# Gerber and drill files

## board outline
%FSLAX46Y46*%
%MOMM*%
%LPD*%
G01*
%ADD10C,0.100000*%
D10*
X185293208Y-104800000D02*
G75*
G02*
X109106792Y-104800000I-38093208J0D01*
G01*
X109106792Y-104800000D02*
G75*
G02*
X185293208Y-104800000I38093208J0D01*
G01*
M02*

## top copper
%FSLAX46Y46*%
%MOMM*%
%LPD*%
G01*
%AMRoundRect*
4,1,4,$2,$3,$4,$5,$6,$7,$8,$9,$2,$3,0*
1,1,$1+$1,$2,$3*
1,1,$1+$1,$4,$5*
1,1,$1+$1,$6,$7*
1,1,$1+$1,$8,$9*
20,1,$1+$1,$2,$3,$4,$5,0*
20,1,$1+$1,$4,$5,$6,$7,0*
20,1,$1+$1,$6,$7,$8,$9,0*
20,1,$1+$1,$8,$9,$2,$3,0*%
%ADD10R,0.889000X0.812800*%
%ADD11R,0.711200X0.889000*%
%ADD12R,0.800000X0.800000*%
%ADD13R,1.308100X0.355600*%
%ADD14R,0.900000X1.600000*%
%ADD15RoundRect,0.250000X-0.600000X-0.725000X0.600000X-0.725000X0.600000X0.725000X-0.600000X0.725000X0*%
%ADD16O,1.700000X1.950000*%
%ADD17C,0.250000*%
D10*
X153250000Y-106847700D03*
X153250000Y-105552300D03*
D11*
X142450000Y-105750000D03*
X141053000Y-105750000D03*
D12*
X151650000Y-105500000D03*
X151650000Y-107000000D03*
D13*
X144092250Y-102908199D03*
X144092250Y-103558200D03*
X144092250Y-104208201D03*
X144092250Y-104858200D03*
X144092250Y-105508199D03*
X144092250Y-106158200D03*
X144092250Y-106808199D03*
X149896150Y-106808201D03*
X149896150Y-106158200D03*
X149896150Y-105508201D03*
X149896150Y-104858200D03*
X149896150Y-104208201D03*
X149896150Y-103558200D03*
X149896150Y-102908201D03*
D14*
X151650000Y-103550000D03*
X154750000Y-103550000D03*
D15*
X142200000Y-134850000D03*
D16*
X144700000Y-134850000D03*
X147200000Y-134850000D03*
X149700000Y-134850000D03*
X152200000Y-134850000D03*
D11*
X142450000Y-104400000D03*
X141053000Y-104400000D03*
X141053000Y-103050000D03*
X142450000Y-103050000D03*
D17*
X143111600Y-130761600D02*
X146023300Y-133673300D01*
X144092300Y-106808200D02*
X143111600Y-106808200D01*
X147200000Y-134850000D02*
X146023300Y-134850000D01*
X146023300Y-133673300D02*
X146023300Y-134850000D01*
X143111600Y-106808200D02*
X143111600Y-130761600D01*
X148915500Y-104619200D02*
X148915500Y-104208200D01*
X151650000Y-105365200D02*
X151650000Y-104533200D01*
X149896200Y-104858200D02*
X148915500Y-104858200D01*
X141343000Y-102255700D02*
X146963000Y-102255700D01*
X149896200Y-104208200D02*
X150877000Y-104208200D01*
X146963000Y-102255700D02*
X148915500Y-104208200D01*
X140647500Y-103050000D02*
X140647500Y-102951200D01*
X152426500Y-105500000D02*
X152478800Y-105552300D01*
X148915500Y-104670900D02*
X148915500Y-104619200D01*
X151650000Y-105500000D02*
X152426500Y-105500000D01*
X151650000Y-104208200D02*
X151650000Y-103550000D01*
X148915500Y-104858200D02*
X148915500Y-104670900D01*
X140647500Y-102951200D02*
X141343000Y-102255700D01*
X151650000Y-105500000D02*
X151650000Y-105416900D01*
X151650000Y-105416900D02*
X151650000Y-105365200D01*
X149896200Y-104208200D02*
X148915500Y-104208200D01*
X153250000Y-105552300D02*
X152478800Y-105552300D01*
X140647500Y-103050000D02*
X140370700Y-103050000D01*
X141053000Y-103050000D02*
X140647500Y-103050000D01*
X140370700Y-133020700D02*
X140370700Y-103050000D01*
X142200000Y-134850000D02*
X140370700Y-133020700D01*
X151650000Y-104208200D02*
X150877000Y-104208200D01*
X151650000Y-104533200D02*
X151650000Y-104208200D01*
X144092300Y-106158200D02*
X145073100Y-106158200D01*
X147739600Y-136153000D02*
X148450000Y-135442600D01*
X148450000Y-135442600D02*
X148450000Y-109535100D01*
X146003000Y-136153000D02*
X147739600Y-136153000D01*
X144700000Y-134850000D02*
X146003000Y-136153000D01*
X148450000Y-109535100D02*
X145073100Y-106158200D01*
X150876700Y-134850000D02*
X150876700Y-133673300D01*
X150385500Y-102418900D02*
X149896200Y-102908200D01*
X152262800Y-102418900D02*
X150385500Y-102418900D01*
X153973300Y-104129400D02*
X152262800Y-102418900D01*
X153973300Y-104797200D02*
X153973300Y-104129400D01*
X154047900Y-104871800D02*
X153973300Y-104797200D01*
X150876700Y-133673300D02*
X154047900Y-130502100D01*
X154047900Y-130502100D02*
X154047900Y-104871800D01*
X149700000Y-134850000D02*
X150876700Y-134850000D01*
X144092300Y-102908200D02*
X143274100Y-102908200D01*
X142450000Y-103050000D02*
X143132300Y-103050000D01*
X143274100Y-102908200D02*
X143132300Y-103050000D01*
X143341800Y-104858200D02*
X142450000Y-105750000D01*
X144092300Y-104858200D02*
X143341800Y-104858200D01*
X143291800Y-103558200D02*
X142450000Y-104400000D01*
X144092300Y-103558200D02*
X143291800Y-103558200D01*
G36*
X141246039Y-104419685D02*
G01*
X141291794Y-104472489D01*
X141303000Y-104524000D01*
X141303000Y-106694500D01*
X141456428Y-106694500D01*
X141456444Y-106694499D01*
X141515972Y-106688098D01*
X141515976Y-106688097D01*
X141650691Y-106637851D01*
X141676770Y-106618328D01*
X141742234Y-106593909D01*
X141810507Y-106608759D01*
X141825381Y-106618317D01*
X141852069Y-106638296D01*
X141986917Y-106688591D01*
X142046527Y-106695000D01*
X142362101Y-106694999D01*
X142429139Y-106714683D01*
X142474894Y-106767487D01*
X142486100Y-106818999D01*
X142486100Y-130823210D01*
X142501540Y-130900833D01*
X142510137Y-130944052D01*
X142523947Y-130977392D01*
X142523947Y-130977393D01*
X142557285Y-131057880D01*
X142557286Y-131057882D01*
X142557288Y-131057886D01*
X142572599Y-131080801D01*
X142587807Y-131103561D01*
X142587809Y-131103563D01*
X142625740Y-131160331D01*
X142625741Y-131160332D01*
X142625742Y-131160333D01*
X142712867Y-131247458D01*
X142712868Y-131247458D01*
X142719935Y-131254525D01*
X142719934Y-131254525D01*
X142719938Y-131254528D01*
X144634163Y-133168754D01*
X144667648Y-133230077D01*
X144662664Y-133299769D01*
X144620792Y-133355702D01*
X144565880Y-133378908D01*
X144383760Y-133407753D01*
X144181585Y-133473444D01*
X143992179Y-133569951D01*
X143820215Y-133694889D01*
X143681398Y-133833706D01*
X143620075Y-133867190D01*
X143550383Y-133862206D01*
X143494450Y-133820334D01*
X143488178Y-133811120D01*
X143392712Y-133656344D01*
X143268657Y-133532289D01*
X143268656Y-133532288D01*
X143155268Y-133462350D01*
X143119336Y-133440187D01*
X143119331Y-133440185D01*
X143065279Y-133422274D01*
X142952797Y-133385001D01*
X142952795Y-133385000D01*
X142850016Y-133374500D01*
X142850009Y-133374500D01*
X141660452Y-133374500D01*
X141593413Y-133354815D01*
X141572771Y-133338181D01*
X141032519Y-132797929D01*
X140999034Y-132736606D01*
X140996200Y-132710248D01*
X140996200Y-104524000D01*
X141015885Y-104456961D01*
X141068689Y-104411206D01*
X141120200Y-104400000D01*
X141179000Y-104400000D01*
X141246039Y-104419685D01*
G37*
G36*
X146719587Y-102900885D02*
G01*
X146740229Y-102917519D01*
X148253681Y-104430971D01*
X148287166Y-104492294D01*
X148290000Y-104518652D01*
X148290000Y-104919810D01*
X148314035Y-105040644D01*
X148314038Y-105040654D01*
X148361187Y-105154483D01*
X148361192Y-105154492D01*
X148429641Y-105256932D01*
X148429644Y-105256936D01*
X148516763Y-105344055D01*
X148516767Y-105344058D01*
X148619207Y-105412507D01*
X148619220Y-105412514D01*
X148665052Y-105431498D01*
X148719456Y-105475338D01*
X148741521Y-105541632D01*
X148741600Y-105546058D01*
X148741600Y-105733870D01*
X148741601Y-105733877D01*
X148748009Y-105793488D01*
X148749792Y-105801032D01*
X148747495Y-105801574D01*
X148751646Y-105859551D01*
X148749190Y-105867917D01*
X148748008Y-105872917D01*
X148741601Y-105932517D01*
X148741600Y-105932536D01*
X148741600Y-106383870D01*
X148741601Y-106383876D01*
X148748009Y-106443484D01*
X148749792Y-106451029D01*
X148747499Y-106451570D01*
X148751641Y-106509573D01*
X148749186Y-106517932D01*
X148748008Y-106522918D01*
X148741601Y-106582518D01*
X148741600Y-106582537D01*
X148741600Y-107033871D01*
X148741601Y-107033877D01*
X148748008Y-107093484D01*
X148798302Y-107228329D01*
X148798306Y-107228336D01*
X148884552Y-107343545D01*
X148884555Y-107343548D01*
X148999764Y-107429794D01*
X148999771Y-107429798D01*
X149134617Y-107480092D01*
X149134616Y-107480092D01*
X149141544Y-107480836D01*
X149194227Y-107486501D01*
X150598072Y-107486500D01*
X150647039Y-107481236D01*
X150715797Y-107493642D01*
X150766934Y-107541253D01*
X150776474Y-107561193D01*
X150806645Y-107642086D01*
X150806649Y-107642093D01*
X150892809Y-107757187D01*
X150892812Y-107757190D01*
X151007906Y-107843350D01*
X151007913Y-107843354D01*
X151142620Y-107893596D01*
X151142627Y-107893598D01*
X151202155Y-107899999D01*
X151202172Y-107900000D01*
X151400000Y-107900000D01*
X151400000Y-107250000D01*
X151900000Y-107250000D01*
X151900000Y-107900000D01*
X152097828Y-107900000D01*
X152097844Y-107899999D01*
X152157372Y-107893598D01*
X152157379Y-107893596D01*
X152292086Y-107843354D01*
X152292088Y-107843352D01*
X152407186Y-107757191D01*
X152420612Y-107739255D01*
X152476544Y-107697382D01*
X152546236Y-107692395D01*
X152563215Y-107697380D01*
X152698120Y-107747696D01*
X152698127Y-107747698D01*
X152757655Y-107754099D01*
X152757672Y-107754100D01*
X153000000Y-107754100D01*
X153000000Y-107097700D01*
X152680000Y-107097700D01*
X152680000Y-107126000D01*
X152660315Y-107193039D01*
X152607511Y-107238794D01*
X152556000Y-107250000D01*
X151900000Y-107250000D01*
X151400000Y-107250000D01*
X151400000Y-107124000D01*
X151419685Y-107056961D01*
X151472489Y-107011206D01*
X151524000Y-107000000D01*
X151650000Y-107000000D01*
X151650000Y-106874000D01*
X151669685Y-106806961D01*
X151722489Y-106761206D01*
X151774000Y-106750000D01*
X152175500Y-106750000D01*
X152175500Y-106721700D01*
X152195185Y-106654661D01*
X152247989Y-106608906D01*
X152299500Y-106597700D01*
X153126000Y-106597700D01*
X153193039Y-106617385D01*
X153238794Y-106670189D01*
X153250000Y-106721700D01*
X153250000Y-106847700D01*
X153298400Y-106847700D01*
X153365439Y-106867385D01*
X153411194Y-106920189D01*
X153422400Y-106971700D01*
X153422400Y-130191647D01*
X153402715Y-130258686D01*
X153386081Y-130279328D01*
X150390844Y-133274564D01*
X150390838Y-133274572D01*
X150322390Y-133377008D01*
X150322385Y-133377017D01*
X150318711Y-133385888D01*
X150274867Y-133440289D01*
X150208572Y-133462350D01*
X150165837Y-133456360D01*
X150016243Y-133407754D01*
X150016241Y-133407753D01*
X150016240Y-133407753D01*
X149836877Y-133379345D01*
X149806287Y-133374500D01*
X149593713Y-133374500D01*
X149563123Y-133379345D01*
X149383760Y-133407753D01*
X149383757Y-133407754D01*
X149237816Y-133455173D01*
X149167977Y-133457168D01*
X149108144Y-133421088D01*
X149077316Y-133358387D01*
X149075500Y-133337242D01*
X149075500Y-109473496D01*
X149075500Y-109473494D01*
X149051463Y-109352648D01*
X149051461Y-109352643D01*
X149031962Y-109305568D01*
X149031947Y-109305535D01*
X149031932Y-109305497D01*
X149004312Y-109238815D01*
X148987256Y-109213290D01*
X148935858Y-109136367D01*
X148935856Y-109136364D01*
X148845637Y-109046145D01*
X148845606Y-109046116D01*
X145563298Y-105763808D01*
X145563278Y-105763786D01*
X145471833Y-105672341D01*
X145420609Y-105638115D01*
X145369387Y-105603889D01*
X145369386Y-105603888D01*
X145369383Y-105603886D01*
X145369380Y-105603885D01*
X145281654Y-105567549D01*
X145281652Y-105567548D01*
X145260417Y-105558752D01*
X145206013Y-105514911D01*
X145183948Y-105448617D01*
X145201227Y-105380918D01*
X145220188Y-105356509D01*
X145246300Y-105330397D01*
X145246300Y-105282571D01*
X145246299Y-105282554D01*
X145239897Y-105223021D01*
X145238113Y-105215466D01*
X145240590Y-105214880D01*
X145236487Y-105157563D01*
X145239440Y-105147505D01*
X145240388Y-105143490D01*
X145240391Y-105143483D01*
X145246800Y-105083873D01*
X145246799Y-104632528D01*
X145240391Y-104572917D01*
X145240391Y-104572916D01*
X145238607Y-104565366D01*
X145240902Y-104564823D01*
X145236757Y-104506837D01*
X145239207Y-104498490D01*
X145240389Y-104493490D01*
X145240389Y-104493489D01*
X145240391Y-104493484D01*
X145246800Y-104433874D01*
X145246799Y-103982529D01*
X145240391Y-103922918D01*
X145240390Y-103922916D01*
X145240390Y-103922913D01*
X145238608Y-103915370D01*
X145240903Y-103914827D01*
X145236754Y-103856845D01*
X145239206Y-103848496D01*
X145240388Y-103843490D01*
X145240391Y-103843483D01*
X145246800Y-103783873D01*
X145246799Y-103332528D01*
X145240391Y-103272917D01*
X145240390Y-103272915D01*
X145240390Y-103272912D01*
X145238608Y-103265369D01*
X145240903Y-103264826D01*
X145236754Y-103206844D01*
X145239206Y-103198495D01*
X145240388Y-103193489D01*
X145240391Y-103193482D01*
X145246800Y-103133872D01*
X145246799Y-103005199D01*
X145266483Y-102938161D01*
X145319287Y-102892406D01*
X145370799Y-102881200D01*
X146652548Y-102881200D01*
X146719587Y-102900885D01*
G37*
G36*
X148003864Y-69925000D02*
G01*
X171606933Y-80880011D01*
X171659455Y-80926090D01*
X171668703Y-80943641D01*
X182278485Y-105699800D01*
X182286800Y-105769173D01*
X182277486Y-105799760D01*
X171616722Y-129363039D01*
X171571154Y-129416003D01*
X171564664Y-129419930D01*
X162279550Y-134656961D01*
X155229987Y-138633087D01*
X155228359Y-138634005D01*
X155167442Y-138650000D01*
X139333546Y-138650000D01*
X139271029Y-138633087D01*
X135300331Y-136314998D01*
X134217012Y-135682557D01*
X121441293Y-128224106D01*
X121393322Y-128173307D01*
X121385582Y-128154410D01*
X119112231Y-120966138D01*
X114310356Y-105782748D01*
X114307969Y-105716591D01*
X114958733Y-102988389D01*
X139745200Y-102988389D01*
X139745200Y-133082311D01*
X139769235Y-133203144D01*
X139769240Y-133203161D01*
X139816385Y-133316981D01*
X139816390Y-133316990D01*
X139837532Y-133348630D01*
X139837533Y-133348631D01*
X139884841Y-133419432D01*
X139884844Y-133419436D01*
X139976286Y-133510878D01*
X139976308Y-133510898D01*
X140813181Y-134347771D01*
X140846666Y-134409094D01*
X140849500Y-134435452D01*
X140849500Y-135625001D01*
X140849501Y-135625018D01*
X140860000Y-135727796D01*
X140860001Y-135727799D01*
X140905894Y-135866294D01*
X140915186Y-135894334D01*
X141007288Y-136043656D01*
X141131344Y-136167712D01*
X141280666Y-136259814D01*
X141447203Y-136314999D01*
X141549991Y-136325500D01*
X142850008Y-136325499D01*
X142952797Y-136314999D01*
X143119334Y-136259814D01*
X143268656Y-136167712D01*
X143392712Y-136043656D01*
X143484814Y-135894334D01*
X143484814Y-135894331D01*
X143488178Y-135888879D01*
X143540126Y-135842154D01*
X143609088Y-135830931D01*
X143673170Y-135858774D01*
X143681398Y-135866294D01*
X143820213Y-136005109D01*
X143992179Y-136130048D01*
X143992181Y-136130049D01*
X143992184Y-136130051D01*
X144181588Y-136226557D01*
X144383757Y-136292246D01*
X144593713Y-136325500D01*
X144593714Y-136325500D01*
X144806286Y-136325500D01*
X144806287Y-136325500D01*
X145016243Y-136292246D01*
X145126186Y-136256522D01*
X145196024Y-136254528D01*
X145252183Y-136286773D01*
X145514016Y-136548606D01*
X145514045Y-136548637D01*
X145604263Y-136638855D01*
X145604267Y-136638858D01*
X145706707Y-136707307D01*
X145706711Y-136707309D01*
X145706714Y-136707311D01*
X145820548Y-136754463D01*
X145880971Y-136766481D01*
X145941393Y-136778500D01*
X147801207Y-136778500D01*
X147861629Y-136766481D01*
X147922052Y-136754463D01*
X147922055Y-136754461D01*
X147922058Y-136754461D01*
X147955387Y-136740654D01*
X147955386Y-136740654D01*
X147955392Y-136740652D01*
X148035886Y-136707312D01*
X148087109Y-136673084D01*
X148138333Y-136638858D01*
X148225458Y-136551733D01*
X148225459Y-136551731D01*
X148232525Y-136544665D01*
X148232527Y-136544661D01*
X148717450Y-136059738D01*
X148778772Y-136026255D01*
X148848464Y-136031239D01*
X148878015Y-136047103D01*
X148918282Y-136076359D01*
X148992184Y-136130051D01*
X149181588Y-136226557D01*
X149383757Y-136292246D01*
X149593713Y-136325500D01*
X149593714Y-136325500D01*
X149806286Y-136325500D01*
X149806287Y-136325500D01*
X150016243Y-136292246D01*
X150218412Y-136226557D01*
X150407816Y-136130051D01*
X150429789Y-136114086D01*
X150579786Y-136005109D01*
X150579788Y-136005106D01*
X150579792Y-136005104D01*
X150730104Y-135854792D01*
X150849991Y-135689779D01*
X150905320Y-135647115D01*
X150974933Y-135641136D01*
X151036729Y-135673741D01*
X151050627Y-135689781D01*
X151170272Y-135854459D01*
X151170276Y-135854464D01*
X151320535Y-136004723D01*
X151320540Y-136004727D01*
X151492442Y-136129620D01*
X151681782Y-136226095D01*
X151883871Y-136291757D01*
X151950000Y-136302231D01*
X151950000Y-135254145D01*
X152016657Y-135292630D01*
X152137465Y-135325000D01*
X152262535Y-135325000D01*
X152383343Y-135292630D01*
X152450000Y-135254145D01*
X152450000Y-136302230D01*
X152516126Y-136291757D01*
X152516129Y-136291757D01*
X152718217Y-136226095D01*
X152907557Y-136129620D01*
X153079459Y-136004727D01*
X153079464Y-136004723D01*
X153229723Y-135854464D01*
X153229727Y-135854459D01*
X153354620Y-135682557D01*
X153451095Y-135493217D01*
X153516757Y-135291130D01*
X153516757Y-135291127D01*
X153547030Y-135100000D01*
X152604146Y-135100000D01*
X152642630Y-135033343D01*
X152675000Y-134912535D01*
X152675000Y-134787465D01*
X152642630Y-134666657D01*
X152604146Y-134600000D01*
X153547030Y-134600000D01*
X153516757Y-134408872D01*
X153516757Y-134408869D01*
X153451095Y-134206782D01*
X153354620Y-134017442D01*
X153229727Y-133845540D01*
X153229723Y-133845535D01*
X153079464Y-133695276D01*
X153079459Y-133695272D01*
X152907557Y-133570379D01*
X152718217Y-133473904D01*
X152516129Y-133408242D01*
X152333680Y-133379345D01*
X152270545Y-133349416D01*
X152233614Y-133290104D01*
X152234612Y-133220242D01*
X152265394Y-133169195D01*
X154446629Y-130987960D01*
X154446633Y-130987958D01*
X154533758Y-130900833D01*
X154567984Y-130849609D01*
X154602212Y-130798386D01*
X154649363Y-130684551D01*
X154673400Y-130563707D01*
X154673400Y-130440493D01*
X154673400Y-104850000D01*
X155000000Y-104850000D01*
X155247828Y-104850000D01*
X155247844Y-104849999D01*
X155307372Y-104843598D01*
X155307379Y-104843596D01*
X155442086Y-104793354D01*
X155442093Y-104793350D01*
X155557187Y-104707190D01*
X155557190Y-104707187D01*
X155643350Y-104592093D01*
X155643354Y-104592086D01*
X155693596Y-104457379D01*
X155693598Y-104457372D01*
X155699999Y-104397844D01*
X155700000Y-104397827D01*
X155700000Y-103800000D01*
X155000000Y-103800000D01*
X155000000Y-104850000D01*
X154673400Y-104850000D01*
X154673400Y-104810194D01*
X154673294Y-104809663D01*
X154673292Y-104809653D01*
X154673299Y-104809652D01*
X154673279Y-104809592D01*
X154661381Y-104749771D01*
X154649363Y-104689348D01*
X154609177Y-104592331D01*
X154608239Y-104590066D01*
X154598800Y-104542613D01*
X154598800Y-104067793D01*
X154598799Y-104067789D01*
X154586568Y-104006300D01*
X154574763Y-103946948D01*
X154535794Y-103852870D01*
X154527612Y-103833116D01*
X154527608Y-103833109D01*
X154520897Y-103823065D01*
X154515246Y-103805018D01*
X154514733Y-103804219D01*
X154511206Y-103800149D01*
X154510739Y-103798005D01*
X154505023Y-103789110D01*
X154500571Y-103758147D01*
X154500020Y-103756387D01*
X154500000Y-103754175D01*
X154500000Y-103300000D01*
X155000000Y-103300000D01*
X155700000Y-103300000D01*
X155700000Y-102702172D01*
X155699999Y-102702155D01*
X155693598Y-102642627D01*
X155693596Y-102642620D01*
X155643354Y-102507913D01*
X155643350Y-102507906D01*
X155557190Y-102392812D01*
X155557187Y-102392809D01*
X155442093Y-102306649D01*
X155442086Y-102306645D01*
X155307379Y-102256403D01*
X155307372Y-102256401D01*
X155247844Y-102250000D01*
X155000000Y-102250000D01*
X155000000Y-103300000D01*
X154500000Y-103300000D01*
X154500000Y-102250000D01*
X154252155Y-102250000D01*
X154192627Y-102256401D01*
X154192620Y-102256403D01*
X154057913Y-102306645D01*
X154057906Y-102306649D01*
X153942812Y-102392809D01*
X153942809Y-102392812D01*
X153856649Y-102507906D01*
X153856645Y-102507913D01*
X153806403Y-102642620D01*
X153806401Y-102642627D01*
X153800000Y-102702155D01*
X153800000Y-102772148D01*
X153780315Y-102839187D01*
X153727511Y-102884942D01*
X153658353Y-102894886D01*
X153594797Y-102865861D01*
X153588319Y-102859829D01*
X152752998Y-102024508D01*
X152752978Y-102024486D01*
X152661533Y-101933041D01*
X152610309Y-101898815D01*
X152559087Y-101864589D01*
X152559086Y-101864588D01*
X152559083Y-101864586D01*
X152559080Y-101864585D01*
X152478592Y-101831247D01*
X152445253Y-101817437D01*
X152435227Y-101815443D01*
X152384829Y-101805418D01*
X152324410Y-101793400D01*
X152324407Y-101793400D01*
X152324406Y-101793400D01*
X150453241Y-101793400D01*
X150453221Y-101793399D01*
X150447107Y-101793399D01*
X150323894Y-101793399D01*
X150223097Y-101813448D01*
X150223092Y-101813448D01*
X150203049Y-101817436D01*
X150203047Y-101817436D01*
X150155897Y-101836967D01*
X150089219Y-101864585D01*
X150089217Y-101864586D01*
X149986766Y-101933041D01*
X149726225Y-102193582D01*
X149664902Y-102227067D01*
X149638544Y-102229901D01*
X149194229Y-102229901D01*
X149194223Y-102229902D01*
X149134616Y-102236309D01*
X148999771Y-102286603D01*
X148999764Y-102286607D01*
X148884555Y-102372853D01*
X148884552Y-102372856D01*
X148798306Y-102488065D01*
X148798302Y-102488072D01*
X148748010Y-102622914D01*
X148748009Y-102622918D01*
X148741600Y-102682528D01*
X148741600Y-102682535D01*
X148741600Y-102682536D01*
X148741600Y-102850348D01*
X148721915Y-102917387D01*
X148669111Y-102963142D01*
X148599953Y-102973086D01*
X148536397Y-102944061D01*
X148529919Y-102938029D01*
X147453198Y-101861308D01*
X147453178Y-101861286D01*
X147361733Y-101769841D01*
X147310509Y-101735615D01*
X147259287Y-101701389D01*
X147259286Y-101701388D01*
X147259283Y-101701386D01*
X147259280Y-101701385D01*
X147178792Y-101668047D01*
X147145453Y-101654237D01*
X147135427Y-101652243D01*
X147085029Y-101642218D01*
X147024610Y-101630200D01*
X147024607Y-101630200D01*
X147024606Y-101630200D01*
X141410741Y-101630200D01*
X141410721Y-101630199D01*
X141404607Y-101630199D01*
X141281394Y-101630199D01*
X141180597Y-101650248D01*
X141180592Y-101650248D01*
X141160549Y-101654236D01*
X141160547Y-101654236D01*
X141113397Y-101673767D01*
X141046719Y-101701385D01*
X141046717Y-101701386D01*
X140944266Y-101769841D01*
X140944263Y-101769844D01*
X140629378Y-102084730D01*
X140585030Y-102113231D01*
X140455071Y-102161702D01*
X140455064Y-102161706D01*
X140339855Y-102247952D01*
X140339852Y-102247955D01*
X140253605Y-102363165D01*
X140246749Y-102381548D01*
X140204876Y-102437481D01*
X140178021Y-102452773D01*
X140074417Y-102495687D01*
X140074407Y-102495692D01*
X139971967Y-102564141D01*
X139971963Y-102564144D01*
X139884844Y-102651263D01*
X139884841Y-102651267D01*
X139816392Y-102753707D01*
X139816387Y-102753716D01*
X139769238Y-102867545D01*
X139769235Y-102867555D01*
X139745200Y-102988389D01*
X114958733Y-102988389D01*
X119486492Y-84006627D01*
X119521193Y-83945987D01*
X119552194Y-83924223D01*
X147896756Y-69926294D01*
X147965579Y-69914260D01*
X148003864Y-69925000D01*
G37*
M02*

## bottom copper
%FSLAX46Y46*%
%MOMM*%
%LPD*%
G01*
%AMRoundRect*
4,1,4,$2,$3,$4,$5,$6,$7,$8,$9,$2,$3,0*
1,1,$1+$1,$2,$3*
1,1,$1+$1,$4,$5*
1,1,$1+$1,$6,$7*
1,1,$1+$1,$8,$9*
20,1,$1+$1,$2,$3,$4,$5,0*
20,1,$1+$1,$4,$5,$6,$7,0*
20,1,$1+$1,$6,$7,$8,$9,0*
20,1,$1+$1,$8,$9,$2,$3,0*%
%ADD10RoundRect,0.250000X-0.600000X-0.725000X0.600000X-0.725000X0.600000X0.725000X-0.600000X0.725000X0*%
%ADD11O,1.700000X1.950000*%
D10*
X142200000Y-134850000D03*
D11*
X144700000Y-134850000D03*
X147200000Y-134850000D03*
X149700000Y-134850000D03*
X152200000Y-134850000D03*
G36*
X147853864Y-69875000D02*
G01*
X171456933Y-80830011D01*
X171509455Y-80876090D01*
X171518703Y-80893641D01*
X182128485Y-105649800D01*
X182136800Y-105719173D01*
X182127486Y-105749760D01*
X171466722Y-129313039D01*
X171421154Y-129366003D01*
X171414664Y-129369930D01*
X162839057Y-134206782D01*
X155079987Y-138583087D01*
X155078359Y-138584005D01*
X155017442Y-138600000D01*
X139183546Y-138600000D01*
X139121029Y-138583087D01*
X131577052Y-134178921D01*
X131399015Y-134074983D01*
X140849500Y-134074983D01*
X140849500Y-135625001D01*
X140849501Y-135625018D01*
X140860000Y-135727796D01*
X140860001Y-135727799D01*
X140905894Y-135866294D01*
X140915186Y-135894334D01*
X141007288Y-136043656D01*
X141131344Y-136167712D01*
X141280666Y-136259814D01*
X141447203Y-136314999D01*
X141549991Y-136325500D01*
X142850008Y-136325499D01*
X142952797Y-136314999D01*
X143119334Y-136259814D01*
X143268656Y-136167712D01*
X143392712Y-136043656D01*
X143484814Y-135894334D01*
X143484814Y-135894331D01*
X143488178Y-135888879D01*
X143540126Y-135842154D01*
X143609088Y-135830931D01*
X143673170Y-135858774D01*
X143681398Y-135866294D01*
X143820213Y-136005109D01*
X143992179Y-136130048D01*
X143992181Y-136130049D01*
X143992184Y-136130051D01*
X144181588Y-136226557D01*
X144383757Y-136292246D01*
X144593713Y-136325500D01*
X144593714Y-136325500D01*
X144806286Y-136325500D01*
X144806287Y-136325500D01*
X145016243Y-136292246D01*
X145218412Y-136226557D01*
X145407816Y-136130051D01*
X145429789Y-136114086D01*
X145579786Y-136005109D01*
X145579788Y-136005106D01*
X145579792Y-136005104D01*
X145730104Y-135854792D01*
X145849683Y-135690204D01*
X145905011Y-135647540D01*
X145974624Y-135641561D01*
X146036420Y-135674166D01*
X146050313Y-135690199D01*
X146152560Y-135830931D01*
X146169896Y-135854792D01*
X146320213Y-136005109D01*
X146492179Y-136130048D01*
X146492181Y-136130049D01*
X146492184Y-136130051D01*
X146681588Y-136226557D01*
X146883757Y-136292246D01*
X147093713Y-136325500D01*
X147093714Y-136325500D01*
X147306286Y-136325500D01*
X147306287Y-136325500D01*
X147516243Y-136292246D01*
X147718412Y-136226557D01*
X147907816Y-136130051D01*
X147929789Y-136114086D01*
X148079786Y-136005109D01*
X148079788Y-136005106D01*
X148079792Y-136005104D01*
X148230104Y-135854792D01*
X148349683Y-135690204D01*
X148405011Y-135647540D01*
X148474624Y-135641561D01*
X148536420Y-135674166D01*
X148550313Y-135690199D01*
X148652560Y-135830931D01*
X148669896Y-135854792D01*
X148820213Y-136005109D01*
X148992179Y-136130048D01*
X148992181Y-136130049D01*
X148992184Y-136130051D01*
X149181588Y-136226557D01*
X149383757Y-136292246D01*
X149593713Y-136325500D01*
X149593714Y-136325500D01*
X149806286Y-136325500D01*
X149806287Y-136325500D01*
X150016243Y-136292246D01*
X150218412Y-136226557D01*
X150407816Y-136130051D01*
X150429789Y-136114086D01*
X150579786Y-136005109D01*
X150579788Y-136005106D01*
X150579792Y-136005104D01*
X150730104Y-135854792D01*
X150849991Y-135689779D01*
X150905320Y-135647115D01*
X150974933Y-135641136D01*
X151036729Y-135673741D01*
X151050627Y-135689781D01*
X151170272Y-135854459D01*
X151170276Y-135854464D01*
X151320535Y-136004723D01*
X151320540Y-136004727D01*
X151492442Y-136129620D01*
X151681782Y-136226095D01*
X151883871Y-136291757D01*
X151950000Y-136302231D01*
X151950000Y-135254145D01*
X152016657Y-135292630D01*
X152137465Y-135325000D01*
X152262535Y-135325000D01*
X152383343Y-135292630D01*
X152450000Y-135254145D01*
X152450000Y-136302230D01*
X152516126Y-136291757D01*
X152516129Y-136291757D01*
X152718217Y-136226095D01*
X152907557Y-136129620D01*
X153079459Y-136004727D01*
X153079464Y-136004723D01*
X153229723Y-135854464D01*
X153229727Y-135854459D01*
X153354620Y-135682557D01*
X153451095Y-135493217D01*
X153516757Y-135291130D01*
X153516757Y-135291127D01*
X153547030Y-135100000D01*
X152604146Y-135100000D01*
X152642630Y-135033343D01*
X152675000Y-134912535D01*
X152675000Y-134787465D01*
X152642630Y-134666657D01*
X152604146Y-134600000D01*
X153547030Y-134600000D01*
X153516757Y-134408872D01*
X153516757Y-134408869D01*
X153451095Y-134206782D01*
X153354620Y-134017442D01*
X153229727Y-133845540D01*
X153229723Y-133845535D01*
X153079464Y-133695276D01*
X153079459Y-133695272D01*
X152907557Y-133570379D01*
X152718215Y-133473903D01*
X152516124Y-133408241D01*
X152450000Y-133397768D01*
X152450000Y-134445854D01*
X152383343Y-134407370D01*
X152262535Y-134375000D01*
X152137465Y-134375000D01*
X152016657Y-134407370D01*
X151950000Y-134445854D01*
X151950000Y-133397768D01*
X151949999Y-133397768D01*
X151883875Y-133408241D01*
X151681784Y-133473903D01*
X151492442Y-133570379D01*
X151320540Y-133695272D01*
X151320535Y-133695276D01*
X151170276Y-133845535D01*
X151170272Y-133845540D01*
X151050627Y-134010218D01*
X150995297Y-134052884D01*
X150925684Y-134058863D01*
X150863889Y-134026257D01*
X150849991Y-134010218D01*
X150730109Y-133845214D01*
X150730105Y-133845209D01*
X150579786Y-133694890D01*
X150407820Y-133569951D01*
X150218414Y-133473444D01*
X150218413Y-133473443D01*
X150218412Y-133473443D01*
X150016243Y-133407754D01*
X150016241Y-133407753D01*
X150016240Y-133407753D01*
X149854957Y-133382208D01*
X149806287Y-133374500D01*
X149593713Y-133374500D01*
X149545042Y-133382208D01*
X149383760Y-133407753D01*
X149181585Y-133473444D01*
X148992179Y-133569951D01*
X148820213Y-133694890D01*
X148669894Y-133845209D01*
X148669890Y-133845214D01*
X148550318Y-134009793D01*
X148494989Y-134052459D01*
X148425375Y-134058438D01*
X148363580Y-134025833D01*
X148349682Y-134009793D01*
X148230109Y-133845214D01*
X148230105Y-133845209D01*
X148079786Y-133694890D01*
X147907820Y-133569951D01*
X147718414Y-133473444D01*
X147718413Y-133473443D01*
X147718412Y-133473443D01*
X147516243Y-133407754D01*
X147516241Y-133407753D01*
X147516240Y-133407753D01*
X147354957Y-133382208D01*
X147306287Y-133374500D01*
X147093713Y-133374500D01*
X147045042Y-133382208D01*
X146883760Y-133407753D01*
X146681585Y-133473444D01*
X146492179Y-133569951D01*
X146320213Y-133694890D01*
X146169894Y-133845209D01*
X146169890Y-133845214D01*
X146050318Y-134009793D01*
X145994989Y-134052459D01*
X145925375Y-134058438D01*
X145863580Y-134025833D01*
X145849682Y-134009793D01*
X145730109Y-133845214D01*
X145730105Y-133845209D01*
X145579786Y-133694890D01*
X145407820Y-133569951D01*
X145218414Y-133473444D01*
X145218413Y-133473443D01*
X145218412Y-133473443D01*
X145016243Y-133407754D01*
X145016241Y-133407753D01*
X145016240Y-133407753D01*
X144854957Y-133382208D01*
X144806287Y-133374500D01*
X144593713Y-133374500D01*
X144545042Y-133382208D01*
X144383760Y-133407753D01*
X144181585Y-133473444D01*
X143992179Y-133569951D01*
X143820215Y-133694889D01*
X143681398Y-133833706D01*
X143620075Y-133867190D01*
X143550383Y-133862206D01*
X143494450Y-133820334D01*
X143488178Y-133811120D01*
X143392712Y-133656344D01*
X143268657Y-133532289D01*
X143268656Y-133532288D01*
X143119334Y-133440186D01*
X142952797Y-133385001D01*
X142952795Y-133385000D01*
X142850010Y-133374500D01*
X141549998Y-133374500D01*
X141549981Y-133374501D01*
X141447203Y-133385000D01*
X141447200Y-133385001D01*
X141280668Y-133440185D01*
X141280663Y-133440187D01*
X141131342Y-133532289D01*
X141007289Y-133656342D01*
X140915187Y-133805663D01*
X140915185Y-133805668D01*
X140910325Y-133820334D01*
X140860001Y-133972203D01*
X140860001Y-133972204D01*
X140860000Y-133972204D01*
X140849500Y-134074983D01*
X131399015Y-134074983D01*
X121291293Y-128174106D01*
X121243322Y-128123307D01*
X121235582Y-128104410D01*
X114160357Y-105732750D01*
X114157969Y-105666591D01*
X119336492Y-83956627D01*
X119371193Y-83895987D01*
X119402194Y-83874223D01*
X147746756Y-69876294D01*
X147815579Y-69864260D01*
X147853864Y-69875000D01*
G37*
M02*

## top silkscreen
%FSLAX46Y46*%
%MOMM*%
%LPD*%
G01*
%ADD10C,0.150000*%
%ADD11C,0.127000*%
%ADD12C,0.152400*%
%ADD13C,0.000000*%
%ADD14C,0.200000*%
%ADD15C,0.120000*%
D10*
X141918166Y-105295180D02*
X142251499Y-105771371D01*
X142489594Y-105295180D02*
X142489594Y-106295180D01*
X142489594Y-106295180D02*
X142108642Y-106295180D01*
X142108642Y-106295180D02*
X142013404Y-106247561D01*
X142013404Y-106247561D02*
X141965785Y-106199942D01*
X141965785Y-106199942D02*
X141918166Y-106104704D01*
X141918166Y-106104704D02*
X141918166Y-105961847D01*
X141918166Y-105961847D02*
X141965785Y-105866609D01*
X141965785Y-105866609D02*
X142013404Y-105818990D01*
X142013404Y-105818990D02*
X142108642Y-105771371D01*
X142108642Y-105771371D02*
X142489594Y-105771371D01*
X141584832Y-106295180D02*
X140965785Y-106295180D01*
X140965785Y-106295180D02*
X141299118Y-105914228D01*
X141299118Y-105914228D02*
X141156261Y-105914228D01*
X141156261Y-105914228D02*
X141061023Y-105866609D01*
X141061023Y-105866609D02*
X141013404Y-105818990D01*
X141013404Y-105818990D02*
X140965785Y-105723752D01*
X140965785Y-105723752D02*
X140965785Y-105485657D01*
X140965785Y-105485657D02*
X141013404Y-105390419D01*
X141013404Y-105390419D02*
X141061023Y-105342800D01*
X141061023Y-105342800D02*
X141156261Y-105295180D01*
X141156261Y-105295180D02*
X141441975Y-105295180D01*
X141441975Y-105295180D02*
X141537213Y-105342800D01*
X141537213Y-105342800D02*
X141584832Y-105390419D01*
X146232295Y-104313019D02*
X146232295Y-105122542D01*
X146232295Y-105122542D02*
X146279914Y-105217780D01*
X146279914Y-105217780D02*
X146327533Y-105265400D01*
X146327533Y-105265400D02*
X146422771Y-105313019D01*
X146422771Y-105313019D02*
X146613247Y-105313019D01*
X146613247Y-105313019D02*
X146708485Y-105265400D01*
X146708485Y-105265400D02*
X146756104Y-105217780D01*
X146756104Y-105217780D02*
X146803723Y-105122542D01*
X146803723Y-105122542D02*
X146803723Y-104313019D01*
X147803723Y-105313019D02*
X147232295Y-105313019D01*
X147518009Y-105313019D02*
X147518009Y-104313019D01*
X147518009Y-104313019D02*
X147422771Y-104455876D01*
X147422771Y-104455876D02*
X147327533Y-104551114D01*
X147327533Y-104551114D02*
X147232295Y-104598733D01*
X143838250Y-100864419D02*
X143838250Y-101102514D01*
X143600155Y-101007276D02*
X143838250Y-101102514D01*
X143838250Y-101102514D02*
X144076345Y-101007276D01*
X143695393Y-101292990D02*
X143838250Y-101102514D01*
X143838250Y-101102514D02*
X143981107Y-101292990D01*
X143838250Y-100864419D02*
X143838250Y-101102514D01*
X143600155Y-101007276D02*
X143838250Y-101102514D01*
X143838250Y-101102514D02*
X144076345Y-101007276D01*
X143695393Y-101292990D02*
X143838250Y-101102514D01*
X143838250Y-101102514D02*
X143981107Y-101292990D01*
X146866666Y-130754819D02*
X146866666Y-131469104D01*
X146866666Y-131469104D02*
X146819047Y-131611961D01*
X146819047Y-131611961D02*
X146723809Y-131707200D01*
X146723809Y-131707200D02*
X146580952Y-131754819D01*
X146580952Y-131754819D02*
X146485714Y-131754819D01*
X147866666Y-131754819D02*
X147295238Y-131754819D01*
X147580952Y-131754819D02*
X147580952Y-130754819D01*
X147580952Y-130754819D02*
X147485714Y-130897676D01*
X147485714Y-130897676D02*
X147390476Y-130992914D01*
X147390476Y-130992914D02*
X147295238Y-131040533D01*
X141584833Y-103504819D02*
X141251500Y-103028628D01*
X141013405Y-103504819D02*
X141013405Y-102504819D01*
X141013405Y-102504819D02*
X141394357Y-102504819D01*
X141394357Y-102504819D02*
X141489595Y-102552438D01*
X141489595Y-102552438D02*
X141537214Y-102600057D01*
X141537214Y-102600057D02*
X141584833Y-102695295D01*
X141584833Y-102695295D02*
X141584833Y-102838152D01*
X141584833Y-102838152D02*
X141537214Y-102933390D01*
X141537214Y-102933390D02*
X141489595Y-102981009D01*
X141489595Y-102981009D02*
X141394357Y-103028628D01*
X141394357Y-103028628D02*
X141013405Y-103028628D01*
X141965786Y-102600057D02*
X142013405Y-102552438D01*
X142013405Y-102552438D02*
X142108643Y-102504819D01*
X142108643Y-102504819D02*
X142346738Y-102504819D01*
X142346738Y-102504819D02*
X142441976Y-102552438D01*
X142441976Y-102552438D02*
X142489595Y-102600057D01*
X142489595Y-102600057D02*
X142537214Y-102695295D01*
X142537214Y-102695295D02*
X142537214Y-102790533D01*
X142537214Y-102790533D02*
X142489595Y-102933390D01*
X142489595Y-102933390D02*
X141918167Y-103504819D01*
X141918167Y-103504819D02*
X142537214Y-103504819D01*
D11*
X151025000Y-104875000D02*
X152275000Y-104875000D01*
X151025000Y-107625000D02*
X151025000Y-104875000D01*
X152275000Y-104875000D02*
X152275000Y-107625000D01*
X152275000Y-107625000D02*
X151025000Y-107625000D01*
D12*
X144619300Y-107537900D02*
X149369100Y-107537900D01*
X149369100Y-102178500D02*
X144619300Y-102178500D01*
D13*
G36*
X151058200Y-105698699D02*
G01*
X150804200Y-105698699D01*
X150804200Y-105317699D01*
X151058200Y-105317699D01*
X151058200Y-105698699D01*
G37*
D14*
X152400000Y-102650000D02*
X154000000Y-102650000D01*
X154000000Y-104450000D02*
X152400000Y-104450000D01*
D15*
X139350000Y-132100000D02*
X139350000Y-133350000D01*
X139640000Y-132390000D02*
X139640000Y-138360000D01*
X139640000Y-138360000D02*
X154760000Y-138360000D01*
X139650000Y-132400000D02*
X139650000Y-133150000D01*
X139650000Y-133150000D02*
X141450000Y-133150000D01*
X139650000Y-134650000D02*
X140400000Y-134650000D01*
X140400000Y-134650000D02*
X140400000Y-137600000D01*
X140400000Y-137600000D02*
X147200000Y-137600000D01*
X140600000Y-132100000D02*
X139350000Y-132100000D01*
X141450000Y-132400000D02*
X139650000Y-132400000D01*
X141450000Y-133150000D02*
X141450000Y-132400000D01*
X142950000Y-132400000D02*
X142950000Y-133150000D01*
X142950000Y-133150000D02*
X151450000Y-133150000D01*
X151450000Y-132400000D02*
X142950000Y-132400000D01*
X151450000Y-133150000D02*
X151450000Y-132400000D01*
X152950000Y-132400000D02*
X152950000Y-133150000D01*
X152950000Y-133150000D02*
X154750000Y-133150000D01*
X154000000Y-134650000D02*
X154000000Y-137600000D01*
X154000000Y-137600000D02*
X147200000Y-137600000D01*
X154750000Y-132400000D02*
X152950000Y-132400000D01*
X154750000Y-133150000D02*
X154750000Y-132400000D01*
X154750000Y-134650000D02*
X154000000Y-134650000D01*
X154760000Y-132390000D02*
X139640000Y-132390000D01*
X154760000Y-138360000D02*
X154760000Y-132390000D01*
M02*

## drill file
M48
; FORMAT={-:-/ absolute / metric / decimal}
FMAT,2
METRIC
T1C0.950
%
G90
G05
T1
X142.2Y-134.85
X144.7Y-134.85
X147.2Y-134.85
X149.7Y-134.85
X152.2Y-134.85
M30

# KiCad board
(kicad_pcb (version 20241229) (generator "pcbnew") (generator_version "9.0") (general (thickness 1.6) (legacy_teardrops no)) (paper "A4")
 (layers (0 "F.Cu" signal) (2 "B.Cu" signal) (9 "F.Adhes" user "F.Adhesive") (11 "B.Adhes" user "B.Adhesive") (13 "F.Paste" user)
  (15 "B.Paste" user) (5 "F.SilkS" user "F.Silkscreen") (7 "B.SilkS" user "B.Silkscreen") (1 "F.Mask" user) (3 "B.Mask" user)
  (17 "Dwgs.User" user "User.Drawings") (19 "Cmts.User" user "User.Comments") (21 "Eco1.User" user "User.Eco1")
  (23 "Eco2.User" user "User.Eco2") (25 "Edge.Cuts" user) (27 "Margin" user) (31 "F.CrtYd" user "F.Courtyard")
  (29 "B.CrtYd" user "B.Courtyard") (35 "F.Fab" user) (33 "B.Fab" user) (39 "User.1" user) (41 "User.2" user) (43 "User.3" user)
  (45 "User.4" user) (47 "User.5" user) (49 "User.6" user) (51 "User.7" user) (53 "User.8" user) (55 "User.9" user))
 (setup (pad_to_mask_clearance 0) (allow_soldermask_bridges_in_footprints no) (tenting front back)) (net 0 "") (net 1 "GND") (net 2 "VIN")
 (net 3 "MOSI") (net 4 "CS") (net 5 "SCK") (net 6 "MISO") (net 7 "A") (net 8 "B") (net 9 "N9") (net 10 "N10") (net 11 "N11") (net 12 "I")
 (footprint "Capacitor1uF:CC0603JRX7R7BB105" (layer "F.Cu") (at 153.25 106.2 90)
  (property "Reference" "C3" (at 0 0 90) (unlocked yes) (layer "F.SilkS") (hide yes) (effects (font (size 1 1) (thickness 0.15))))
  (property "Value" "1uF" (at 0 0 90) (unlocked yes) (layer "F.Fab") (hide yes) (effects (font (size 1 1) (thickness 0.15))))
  (pad "1" smd rect (at -0.6477 0 90) (size 0.8128 0.889) (layers "F.Cu" "F.Mask" "F.Paste") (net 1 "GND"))
  (pad "2" smd rect (at 0.6477 0 90) (size 0.8128 0.889) (layers "F.Cu" "F.Mask" "F.Paste") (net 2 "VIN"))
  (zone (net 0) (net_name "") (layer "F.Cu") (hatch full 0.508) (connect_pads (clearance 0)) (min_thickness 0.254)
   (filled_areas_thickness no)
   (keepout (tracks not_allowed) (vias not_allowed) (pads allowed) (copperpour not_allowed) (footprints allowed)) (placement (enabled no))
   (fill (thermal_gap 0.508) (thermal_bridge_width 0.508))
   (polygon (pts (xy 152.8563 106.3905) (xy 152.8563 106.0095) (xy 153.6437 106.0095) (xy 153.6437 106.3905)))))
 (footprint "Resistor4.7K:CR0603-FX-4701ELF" (layer "F.Cu") (at 141.7515 105.75 180)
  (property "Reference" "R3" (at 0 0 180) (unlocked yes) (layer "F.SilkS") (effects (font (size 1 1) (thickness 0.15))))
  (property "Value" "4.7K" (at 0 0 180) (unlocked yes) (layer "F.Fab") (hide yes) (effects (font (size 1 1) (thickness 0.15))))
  (pad "1" smd rect (at -0.6985 0 180) (size 0.7112 0.889) (layers "F.Cu" "F.Mask" "F.Paste") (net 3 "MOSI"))
  (pad "2" smd rect (at 0.6985 0 180) (size 0.7112 0.889) (layers "F.Cu" "F.Mask" "F.Paste") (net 1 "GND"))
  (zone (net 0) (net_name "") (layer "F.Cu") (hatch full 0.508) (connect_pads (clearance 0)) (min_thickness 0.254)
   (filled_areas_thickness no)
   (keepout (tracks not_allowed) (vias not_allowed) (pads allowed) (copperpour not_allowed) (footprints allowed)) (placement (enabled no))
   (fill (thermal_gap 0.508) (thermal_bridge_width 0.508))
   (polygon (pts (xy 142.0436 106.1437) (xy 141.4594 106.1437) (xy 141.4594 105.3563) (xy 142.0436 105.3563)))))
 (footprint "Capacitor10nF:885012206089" (layer "F.Cu") (at 151.65 106.25 -90)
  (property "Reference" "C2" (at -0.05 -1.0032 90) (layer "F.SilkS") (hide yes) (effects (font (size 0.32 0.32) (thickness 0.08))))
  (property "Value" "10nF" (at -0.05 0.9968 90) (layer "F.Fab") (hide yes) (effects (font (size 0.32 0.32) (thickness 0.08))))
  (fp_line (start -1.375 0.625) (end -1.375 -0.625) (stroke (width 0.127) (type solid)) (layer "F.SilkS"))
  (fp_line (start 1.375 0.625) (end -1.375 0.625) (stroke (width 0.127) (type solid)) (layer "F.SilkS"))
  (fp_line (start -1.375 -0.625) (end 1.375 -0.625) (stroke (width 0.127) (type solid)) (layer "F.SilkS"))
  (fp_line (start 1.375 -0.625) (end 1.375 0.625) (stroke (width 0.127) (type solid)) (layer "F.SilkS"))
  (pad "1" smd rect (at -0.75 0 270) (size 0.8 0.8) (layers "F.Cu" "F.Mask" "F.Paste") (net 2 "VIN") (solder_mask_margin 0.102))
  (pad "2" smd rect (at 0.75 0 270) (size 0.8 0.8) (layers "F.Cu" "F.Mask" "F.Paste") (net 1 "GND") (solder_mask_margin 0.102)))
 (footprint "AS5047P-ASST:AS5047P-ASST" (layer "F.Cu") (at 146.9942 104.8582)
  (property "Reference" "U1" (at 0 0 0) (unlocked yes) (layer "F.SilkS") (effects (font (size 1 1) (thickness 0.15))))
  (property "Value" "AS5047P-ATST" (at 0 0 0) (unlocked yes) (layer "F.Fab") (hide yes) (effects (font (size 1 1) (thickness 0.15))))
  (fp_line (start -2.3749 2.6797) (end 2.3749 2.6797) (stroke (width 0.1524) (type solid)) (layer "F.SilkS"))
  (fp_line (start 2.3749 -2.6797) (end -2.3749 -2.6797) (stroke (width 0.1524) (type solid)) (layer "F.SilkS"))
  (fp_poly
   (pts (xy 4.064 0.459499) (xy 4.064 0.840499) (xy 3.81 0.840499) (xy 3.81 0.459499)) (stroke (width 0) (type solid)) (fill yes)
   (layer "F.SilkS"))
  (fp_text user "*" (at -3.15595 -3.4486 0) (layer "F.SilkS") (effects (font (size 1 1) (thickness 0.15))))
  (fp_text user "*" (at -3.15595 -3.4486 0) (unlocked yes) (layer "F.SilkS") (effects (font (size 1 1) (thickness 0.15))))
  (pad "1" smd rect (at -2.90195 -1.950001) (size 1.3081 0.3556) (layers "F.Cu" "F.Mask" "F.Paste") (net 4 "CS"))
  (pad "2" smd rect (at -2.90195 -1.3) (size 1.3081 0.3556) (layers "F.Cu" "F.Mask" "F.Paste") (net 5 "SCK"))
  (pad "3" smd rect (at -2.90195 -0.649999) (size 1.3081 0.3556) (layers "F.Cu" "F.Mask" "F.Paste") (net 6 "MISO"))
  (pad "4" smd rect (at -2.90195 0) (size 1.3081 0.3556) (layers "F.Cu" "F.Mask" "F.Paste") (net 3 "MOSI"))
  (pad "5" smd rect (at -2.90195 0.649999) (size 1.3081 0.3556) (layers "F.Cu" "F.Mask" "F.Paste") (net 1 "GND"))
  (pad "6" smd rect (at -2.90195 1.3) (size 1.3081 0.3556) (layers "F.Cu" "F.Mask" "F.Paste") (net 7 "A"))
  (pad "7" smd rect (at -2.90195 1.949999) (size 1.3081 0.3556) (layers "F.Cu" "F.Mask" "F.Paste") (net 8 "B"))
  (pad "8" smd rect (at 2.90195 1.950001) (size 1.3081 0.3556) (layers "F.Cu" "F.Mask" "F.Paste") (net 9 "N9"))
  (pad "9" smd rect (at 2.90195 1.3) (size 1.3081 0.3556) (layers "F.Cu" "F.Mask" "F.Paste") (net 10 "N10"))
  (pad "10" smd rect (at 2.90195 0.650001) (size 1.3081 0.3556) (layers "F.Cu" "F.Mask" "F.Paste") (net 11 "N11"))
  (pad "11" smd rect (at 2.90195 0) (size 1.3081 0.3556) (layers "F.Cu" "F.Mask" "F.Paste") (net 2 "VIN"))
  (pad "12" smd rect (at 2.90195 -0.649999) (size 1.3081 0.3556) (layers "F.Cu" "F.Mask" "F.Paste") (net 2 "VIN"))
  (pad "13" smd rect (at 2.90195 -1.3) (size 1.3081 0.3556) (layers "F.Cu" "F.Mask" "F.Paste") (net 1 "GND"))
  (pad "14" smd rect (at 2.90195 -1.949999) (size 1.3081 0.3556) (layers "F.Cu" "F.Mask" "F.Paste") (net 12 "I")))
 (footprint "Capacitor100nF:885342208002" (layer "F.Cu") (at 153.2 103.55)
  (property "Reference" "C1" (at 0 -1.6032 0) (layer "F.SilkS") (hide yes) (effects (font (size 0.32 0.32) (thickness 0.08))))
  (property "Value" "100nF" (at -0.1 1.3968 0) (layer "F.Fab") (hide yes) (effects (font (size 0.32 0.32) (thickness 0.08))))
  (fp_line (start -0.8 -0.9) (end 0.8 -0.9) (stroke (width 0.2) (type solid)) (layer "F.SilkS"))
  (fp_line (start 0.8 0.9) (end -0.8 0.9) (stroke (width 0.2) (type solid)) (layer "F.SilkS"))
  (pad "1" smd rect (at -1.55 0) (size 0.9 1.6) (layers "F.Cu" "F.Mask" "F.Paste") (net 2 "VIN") (solder_mask_margin 0.102))
  (pad "2" smd rect (at 1.55 0) (size 0.9 1.6) (layers "F.Cu" "F.Mask" "F.Paste") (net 1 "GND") (solder_mask_margin 0.102)))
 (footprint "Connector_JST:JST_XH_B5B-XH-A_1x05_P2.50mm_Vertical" (layer "F.Cu") (at 142.2 134.85)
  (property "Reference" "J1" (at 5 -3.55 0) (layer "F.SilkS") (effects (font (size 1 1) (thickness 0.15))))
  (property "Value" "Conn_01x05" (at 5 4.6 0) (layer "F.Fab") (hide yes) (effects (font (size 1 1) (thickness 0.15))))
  (fp_line (start -2.85 -2.75) (end -2.85 -1.5) (stroke (width 0.12) (type solid)) (layer "F.SilkS"))
  (fp_line (start -2.56 -2.46) (end -2.56 3.51) (stroke (width 0.12) (type solid)) (layer "F.SilkS"))
  (fp_line (start -2.56 3.51) (end 12.56 3.51) (stroke (width 0.12) (type solid)) (layer "F.SilkS"))
  (fp_line (start -2.55 -2.45) (end -2.55 -1.7) (stroke (width 0.12) (type solid)) (layer "F.SilkS"))
  (fp_line (start -2.55 -1.7) (end -0.75 -1.7) (stroke (width 0.12) (type solid)) (layer "F.SilkS"))
  (fp_line (start -2.55 -0.2) (end -1.8 -0.2) (stroke (width 0.12) (type solid)) (layer "F.SilkS"))
  (fp_line (start -1.8 -0.2) (end -1.8 2.75) (stroke (width 0.12) (type solid)) (layer "F.SilkS"))
  (fp_line (start -1.8 2.75) (end 5 2.75) (stroke (width 0.12) (type solid)) (layer "F.SilkS"))
  (fp_line (start -1.6 -2.75) (end -2.85 -2.75) (stroke (width 0.12) (type solid)) (layer "F.SilkS"))
  (fp_line (start -0.75 -2.45) (end -2.55 -2.45) (stroke (width 0.12) (type solid)) (layer "F.SilkS"))
  (fp_line (start -0.75 -1.7) (end -0.75 -2.45) (stroke (width 0.12) (type solid)) (layer "F.SilkS"))
  (fp_line (start 0.75 -2.45) (end 0.75 -1.7) (stroke (width 0.12) (type solid)) (layer "F.SilkS"))
  (fp_line (start 0.75 -1.7) (end 9.25 -1.7) (stroke (width 0.12) (type solid)) (layer "F.SilkS"))
  (fp_line (start 9.25 -2.45) (end 0.75 -2.45) (stroke (width 0.12) (type solid)) (layer "F.SilkS"))
  (fp_line (start 9.25 -1.7) (end 9.25 -2.45) (stroke (width 0.12) (type solid)) (layer "F.SilkS"))
  (fp_line (start 10.75 -2.45) (end 10.75 -1.7) (stroke (width 0.12) (type solid)) (layer "F.SilkS"))
  (fp_line (start 10.75 -1.7) (end 12.55 -1.7) (stroke (width 0.12) (type solid)) (layer "F.SilkS"))
  (fp_line (start 11.8 -0.2) (end 11.8 2.75) (stroke (width 0.12) (type solid)) (layer "F.SilkS"))
  (fp_line (start 11.8 2.75) (end 5 2.75) (stroke (width 0.12) (type solid)) (layer "F.SilkS"))
  (fp_line (start 12.55 -2.45) (end 10.75 -2.45) (stroke (width 0.12) (type solid)) (layer "F.SilkS"))
  (fp_line (start 12.55 -1.7) (end 12.55 -2.45) (stroke (width 0.12) (type solid)) (layer "F.SilkS"))
  (fp_line (start 12.55 -0.2) (end 11.8 -0.2) (stroke (width 0.12) (type solid)) (layer "F.SilkS"))
  (fp_line (start 12.56 -2.46) (end -2.56 -2.46) (stroke (width 0.12) (type solid)) (layer "F.SilkS"))
  (fp_line (start 12.56 3.51) (end 12.56 -2.46) (stroke (width 0.12) (type solid)) (layer "F.SilkS"))
  (pad "1" thru_hole roundrect (at 0 0) (size 1.7 1.95) (drill 0.95) (layers "*.Cu" "*.Mask") (remove_unused_layers no)
   (roundrect_rratio 0.147059) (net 2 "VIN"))
  (pad "2" thru_hole oval (at 2.5 0) (size 1.7 1.95) (drill 0.95) (layers "*.Cu" "*.Mask") (remove_unused_layers no) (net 7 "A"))
  (pad "3" thru_hole oval (at 5 0) (size 1.7 1.95) (drill 0.95) (layers "*.Cu" "*.Mask") (remove_unused_layers no) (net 8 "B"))
  (pad "4" thru_hole oval (at 7.5 0) (size 1.7 1.95) (drill 0.95) (layers "*.Cu" "*.Mask") (remove_unused_layers no) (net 12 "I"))
  (pad "5" thru_hole oval (at 10 0) (size 1.7 1.95) (drill 0.95) (layers "*.Cu" "*.Mask") (remove_unused_layers no) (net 1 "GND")))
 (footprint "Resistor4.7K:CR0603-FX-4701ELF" (layer "F.Cu") (at 141.7515 104.4 180)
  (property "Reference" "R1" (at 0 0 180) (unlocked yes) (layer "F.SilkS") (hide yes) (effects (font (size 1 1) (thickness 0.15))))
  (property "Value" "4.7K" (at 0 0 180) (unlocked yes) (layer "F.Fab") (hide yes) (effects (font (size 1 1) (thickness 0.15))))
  (pad "1" smd rect (at -0.6985 0 180) (size 0.7112 0.889) (layers "F.Cu" "F.Mask" "F.Paste") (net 5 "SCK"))
  (pad "2" smd rect (at 0.6985 0 180) (size 0.7112 0.889) (layers "F.Cu" "F.Mask" "F.Paste") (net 1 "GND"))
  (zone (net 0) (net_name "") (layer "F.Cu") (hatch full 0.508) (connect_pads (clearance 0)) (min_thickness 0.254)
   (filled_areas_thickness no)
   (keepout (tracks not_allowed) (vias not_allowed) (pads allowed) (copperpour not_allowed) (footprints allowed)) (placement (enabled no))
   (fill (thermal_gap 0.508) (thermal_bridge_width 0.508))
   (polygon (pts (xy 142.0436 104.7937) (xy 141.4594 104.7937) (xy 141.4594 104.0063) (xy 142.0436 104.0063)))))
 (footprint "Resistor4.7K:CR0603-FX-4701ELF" (layer "F.Cu") (at 141.7515 103.05)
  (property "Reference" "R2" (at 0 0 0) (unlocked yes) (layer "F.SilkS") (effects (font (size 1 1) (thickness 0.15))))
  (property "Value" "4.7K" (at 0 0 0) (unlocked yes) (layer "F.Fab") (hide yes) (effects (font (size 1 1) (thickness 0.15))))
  (pad "1" smd rect (at -0.6985 0) (size 0.7112 0.889) (layers "F.Cu" "F.Mask" "F.Paste") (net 2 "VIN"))
  (pad "2" smd rect (at 0.6985 0) (size 0.7112 0.889) (layers "F.Cu" "F.Mask" "F.Paste") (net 4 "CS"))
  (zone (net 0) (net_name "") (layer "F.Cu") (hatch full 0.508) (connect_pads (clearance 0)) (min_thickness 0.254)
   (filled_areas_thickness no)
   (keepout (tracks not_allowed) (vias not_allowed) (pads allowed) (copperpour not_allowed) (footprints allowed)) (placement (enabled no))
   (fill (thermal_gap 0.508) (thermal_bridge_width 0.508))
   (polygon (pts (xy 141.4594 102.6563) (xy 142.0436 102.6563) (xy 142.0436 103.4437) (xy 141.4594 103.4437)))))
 (gr_circle (center 147.2 104.8) (end 183.5 116.35) (stroke (width 0.1) (type default)) (fill no) (layer "Edge.Cuts"))
 (segment (start 143.1116 130.7616) (end 146.0233 133.6733) (width 0.25) (layer "F.Cu") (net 8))
 (segment (start 144.0923 106.8082) (end 143.1116 106.8082) (width 0.25) (layer "F.Cu") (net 8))
 (segment (start 147.2 134.85) (end 146.0233 134.85) (width 0.25) (layer "F.Cu") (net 8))
 (segment (start 146.0233 133.6733) (end 146.0233 134.85) (width 0.25) (layer "F.Cu") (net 8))
 (segment (start 143.1116 106.8082) (end 143.1116 130.7616) (width 0.25) (layer "F.Cu") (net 8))
 (segment (start 148.9155 104.6192) (end 148.9155 104.2082) (width 0.25) (layer "F.Cu") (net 2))
 (segment (start 151.65 105.3652) (end 151.65 104.5332) (width 0.25) (layer "F.Cu") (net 2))
 (segment (start 149.8962 104.8582) (end 148.9155 104.8582) (width 0.25) (layer "F.Cu") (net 2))
 (segment (start 141.343 102.2557) (end 146.963 102.2557) (width 0.25) (layer "F.Cu") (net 2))
 (segment (start 149.8962 104.2082) (end 150.877 104.2082) (width 0.25) (layer "F.Cu") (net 2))
 (segment (start 146.963 102.2557) (end 148.9155 104.2082) (width 0.25) (layer "F.Cu") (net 2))
 (segment (start 140.6475 103.05) (end 140.6475 102.9512) (width 0.25) (layer "F.Cu") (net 2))
 (segment (start 152.4265 105.5) (end 152.4788 105.5523) (width 0.25) (layer "F.Cu") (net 2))
 (segment (start 148.9155 104.6709) (end 148.9155 104.6192) (width 0.25) (layer "F.Cu") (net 2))
 (segment (start 151.65 105.5) (end 152.4265 105.5) (width 0.25) (layer "F.Cu") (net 2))
 (segment (start 151.65 104.2082) (end 151.65 103.55) (width 0.25) (layer "F.Cu") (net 2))
 (segment (start 148.9155 104.8582) (end 148.9155 104.6709) (width 0.25) (layer "F.Cu") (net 2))
 (segment (start 140.6475 102.9512) (end 141.343 102.2557) (width 0.25) (layer "F.Cu") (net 2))
 (segment (start 151.65 105.5) (end 151.65 105.4169) (width 0.25) (layer "F.Cu") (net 2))
 (segment (start 151.65 105.4169) (end 151.65 105.3652) (width 0.25) (layer "F.Cu") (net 2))
 (segment (start 149.8962 104.2082) (end 148.9155 104.2082) (width 0.25) (layer "F.Cu") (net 2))
 (segment (start 153.25 105.5523) (end 152.4788 105.5523) (width 0.25) (layer "F.Cu") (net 2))
 (segment (start 140.6475 103.05) (end 140.3707 103.05) (width 0.25) (layer "F.Cu") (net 2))
 (segment (start 141.053 103.05) (end 140.6475 103.05) (width 0.25) (layer "F.Cu") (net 2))
 (segment (start 140.3707 133.0207) (end 140.3707 103.05) (width 0.25) (layer "F.Cu") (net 2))
 (segment (start 142.2 134.85) (end 140.3707 133.0207) (width 0.25) (layer "F.Cu") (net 2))
 (segment (start 151.65 104.2082) (end 150.877 104.2082) (width 0.25) (layer "F.Cu") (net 2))
 (segment (start 151.65 104.5332) (end 151.65 104.2082) (width 0.25) (layer "F.Cu") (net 2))
 (segment (start 144.0923 106.1582) (end 145.0731 106.1582) (width 0.25) (layer "F.Cu") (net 7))
 (segment (start 147.7396 136.153) (end 148.45 135.4426) (width 0.25) (layer "F.Cu") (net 7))
 (segment (start 148.45 135.4426) (end 148.45 109.5351) (width 0.25) (layer "F.Cu") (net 7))
 (segment (start 146.003 136.153) (end 147.7396 136.153) (width 0.25) (layer "F.Cu") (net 7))
 (segment (start 144.7 134.85) (end 146.003 136.153) (width 0.25) (layer "F.Cu") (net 7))
 (segment (start 148.45 109.5351) (end 145.0731 106.1582) (width 0.25) (layer "F.Cu") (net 7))
 (segment (start 150.8767 134.85) (end 150.8767 133.6733) (width 0.25) (layer "F.Cu") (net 12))
 (segment (start 150.3855 102.4189) (end 149.8962 102.9082) (width 0.25) (layer "F.Cu") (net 12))
 (segment (start 152.2628 102.4189) (end 150.3855 102.4189) (width 0.25) (layer "F.Cu") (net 12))
 (segment (start 153.9733 104.1294) (end 152.2628 102.4189) (width 0.25) (layer "F.Cu") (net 12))
 (segment (start 153.9733 104.7972) (end 153.9733 104.1294) (width 0.25) (layer "F.Cu") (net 12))
 (segment (start 154.0479 104.8718) (end 153.9733 104.7972) (width 0.25) (layer "F.Cu") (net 12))
 (segment (start 150.8767 133.6733) (end 154.0479 130.5021) (width 0.25) (layer "F.Cu") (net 12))
 (segment (start 154.0479 130.5021) (end 154.0479 104.8718) (width 0.25) (layer "F.Cu") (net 12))
 (segment (start 149.7 134.85) (end 150.8767 134.85) (width 0.25) (layer "F.Cu") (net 12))
 (segment (start 144.0923 102.9082) (end 143.2741 102.9082) (width 0.25) (layer "F.Cu") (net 4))
 (segment (start 142.45 103.05) (end 143.1323 103.05) (width 0.25) (layer "F.Cu") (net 4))
 (segment (start 143.2741 102.9082) (end 143.1323 103.05) (width 0.25) (layer "F.Cu") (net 4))
 (segment (start 143.3418 104.8582) (end 142.45 105.75) (width 0.25) (layer "F.Cu") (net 3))
 (segment (start 144.0923 104.8582) (end 143.3418 104.8582) (width 0.25) (layer "F.Cu") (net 3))
 (segment (start 143.2918 103.5582) (end 142.45 104.4) (width 0.25) (layer "F.Cu") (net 5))
 (segment (start 144.0923 103.5582) (end 143.2918 103.5582) (width 0.25) (layer "F.Cu") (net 5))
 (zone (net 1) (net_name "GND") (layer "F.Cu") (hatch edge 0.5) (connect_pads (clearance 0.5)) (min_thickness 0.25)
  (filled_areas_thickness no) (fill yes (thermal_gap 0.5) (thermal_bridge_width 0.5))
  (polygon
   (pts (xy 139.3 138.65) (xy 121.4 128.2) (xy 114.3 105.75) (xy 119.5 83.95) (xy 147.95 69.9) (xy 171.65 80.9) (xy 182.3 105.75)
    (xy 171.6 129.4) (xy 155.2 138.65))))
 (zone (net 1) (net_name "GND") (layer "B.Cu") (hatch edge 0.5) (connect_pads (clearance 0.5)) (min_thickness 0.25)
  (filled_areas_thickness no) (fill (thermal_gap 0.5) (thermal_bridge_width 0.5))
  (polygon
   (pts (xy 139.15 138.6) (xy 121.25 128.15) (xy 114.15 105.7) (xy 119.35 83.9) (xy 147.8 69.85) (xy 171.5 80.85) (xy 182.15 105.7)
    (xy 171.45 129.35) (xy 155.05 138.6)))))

